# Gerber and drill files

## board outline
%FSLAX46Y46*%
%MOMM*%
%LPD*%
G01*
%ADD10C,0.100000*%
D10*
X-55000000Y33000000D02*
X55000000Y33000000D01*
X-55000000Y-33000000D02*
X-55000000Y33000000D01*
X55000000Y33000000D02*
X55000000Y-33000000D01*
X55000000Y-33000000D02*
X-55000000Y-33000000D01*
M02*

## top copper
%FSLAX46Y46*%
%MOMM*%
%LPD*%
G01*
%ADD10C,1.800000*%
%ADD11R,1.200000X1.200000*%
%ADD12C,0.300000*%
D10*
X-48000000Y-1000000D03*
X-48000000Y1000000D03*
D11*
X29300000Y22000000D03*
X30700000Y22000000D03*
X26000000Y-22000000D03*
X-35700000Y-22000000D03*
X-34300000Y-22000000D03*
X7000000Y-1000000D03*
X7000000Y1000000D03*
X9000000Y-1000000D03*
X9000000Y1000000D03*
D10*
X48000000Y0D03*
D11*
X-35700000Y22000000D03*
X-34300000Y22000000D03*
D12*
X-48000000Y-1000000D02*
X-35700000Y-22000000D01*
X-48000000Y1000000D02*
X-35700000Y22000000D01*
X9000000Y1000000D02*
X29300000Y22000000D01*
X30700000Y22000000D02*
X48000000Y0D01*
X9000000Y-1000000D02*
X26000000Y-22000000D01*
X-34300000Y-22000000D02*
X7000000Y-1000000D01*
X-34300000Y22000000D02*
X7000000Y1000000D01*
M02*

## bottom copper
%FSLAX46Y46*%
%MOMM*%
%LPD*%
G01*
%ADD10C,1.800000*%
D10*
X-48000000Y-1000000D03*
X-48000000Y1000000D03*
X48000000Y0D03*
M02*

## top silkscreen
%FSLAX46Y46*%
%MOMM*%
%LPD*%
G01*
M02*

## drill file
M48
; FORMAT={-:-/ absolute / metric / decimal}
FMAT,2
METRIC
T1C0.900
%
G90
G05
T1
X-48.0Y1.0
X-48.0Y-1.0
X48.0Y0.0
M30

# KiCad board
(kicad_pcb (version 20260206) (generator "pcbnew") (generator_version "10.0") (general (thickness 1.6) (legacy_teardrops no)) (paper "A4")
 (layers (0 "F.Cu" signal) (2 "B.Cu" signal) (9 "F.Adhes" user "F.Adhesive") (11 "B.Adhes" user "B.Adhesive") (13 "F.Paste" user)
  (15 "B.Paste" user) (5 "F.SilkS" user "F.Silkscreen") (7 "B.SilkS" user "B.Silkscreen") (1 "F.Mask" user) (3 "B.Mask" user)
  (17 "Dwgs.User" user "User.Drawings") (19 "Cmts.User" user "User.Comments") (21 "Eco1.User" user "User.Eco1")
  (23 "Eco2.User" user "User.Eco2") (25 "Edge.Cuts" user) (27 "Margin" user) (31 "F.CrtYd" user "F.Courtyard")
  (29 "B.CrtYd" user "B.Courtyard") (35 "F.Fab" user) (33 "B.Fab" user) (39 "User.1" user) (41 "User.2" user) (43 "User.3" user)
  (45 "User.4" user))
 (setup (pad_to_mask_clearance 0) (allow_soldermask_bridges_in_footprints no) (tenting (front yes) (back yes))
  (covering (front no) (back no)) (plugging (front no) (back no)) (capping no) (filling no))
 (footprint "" (layer "F.Cu") (at -48 0)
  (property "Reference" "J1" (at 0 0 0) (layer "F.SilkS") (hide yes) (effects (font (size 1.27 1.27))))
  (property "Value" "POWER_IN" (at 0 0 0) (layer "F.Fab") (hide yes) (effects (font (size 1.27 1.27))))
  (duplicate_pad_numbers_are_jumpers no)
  (pad "1" thru_hole circle (at 0 1) (size 1.8 1.8) (drill 0.9) (layers "*.Cu" "*.Mask") (remove_unused_layers no) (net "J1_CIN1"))
  (pad "2" thru_hole circle (at 0 -1) (size 1.8 1.8) (drill 0.9) (layers "*.Cu" "*.Mask") (remove_unused_layers no) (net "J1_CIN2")))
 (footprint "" (layer "F.Cu") (at 30 -22)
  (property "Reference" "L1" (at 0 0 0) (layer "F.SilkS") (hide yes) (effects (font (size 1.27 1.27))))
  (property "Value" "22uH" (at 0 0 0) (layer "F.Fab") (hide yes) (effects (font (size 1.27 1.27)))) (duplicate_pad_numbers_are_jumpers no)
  (pad "1" smd rect (at -0.7 0) (size 1.2 1.2) (layers "F.Cu" "F.Mask" "F.Paste") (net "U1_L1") (thermal_bridge_angle 45))
  (pad "2" smd rect (at 0.7 0) (size 1.2 1.2) (layers "F.Cu" "F.Mask" "F.Paste") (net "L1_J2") (thermal_bridge_angle 45)))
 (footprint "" (layer "F.Cu") (at 26 22)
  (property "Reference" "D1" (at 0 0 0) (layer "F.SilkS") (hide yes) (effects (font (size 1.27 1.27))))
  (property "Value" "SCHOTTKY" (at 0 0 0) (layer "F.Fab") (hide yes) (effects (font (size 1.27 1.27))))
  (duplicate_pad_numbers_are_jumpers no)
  (pad "1" smd rect (at 0 0) (size 1.2 1.2) (layers "F.Cu" "F.Mask" "F.Paste") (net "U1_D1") (thermal_bridge_angle 45)))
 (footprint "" (layer "F.Cu") (at -35 22)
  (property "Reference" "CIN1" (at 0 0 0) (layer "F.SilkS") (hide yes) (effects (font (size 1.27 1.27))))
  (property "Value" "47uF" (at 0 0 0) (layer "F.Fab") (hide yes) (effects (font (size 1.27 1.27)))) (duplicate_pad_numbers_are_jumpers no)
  (pad "1" smd rect (at -0.7 0) (size 1.2 1.2) (layers "F.Cu" "F.Mask" "F.Paste") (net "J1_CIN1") (thermal_bridge_angle 45))
  (pad "2" smd rect (at 0.7 0) (size 1.2 1.2) (layers "F.Cu" "F.Mask" "F.Paste") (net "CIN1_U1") (thermal_bridge_angle 45)))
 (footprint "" (layer "F.Cu") (at 8 0)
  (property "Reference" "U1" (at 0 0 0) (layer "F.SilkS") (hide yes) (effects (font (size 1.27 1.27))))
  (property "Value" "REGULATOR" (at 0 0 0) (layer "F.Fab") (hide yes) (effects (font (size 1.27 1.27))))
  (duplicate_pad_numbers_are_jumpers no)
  (pad "1" smd rect (at -1 1) (size 1.2 1.2) (layers "F.Cu" "F.Mask" "F.Paste") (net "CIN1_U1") (thermal_bridge_angle 45))
  (pad "2" smd rect (at -1 -1) (size 1.2 1.2) (layers "F.Cu" "F.Mask" "F.Paste") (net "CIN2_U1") (thermal_bridge_angle 45))
  (pad "3" smd rect (at 1 1) (size 1.2 1.2) (layers "F.Cu" "F.Mask" "F.Paste") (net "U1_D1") (thermal_bridge_angle 45))
  (pad "4" smd rect (at 1 -1) (size 1.2 1.2) (layers "F.Cu" "F.Mask" "F.Paste") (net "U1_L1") (thermal_bridge_angle 45)))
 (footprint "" (layer "F.Cu") (at 48 0)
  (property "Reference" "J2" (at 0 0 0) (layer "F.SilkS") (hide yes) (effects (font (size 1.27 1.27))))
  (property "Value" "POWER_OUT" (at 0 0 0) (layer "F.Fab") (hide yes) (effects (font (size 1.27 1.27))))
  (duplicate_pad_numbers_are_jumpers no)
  (pad "1" thru_hole circle (at 0 0) (size 1.8 1.8) (drill 0.9) (layers "*.Cu" "*.Mask") (remove_unused_layers no) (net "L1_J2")))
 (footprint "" (layer "F.Cu") (at -35 -22)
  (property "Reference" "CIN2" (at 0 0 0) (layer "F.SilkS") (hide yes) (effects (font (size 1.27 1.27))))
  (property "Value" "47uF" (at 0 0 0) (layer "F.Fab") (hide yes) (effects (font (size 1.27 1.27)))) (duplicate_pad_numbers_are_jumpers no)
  (pad "1" smd rect (at -0.7 0) (size 1.2 1.2) (layers "F.Cu" "F.Mask" "F.Paste") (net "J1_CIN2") (thermal_bridge_angle 45))
  (pad "2" smd rect (at 0.7 0) (size 1.2 1.2) (layers "F.Cu" "F.Mask" "F.Paste") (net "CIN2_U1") (thermal_bridge_angle 45)))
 (gr_line (start -55 -33) (end 55 -33) (stroke (width 0.1) (type default)) (layer "Edge.Cuts"))
 (gr_line (start -55 33) (end -55 -33) (stroke (width 0.1) (type default)) (layer "Edge.Cuts"))
 (gr_line (start 55 -33) (end 55 33) (stroke (width 0.1) (type default)) (layer "Edge.Cuts"))
 (gr_line (start 55 33) (end -55 33) (stroke (width 0.1) (type default)) (layer "Edge.Cuts"))
 (segment (start -48 1) (end -35.7 22) (width 0.3) (layer "F.Cu") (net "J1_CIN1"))
 (segment (start -48 -1) (end -35.7 -22) (width 0.3) (layer "F.Cu") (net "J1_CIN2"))
 (segment (start 9 -1) (end 29.3 -22) (width 0.3) (layer "F.Cu") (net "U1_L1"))
 (segment (start 30.7 -22) (end 48 0) (width 0.3) (layer "F.Cu") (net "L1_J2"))
 (segment (start 9 1) (end 26 22) (width 0.3) (layer "F.Cu") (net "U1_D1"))
 (segment (start -34.3 22) (end 7 1) (width 0.3) (layer "F.Cu") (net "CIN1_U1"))
 (segment (start -34.3 -22) (end 7 -1) (width 0.3) (layer "F.Cu") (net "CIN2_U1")))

